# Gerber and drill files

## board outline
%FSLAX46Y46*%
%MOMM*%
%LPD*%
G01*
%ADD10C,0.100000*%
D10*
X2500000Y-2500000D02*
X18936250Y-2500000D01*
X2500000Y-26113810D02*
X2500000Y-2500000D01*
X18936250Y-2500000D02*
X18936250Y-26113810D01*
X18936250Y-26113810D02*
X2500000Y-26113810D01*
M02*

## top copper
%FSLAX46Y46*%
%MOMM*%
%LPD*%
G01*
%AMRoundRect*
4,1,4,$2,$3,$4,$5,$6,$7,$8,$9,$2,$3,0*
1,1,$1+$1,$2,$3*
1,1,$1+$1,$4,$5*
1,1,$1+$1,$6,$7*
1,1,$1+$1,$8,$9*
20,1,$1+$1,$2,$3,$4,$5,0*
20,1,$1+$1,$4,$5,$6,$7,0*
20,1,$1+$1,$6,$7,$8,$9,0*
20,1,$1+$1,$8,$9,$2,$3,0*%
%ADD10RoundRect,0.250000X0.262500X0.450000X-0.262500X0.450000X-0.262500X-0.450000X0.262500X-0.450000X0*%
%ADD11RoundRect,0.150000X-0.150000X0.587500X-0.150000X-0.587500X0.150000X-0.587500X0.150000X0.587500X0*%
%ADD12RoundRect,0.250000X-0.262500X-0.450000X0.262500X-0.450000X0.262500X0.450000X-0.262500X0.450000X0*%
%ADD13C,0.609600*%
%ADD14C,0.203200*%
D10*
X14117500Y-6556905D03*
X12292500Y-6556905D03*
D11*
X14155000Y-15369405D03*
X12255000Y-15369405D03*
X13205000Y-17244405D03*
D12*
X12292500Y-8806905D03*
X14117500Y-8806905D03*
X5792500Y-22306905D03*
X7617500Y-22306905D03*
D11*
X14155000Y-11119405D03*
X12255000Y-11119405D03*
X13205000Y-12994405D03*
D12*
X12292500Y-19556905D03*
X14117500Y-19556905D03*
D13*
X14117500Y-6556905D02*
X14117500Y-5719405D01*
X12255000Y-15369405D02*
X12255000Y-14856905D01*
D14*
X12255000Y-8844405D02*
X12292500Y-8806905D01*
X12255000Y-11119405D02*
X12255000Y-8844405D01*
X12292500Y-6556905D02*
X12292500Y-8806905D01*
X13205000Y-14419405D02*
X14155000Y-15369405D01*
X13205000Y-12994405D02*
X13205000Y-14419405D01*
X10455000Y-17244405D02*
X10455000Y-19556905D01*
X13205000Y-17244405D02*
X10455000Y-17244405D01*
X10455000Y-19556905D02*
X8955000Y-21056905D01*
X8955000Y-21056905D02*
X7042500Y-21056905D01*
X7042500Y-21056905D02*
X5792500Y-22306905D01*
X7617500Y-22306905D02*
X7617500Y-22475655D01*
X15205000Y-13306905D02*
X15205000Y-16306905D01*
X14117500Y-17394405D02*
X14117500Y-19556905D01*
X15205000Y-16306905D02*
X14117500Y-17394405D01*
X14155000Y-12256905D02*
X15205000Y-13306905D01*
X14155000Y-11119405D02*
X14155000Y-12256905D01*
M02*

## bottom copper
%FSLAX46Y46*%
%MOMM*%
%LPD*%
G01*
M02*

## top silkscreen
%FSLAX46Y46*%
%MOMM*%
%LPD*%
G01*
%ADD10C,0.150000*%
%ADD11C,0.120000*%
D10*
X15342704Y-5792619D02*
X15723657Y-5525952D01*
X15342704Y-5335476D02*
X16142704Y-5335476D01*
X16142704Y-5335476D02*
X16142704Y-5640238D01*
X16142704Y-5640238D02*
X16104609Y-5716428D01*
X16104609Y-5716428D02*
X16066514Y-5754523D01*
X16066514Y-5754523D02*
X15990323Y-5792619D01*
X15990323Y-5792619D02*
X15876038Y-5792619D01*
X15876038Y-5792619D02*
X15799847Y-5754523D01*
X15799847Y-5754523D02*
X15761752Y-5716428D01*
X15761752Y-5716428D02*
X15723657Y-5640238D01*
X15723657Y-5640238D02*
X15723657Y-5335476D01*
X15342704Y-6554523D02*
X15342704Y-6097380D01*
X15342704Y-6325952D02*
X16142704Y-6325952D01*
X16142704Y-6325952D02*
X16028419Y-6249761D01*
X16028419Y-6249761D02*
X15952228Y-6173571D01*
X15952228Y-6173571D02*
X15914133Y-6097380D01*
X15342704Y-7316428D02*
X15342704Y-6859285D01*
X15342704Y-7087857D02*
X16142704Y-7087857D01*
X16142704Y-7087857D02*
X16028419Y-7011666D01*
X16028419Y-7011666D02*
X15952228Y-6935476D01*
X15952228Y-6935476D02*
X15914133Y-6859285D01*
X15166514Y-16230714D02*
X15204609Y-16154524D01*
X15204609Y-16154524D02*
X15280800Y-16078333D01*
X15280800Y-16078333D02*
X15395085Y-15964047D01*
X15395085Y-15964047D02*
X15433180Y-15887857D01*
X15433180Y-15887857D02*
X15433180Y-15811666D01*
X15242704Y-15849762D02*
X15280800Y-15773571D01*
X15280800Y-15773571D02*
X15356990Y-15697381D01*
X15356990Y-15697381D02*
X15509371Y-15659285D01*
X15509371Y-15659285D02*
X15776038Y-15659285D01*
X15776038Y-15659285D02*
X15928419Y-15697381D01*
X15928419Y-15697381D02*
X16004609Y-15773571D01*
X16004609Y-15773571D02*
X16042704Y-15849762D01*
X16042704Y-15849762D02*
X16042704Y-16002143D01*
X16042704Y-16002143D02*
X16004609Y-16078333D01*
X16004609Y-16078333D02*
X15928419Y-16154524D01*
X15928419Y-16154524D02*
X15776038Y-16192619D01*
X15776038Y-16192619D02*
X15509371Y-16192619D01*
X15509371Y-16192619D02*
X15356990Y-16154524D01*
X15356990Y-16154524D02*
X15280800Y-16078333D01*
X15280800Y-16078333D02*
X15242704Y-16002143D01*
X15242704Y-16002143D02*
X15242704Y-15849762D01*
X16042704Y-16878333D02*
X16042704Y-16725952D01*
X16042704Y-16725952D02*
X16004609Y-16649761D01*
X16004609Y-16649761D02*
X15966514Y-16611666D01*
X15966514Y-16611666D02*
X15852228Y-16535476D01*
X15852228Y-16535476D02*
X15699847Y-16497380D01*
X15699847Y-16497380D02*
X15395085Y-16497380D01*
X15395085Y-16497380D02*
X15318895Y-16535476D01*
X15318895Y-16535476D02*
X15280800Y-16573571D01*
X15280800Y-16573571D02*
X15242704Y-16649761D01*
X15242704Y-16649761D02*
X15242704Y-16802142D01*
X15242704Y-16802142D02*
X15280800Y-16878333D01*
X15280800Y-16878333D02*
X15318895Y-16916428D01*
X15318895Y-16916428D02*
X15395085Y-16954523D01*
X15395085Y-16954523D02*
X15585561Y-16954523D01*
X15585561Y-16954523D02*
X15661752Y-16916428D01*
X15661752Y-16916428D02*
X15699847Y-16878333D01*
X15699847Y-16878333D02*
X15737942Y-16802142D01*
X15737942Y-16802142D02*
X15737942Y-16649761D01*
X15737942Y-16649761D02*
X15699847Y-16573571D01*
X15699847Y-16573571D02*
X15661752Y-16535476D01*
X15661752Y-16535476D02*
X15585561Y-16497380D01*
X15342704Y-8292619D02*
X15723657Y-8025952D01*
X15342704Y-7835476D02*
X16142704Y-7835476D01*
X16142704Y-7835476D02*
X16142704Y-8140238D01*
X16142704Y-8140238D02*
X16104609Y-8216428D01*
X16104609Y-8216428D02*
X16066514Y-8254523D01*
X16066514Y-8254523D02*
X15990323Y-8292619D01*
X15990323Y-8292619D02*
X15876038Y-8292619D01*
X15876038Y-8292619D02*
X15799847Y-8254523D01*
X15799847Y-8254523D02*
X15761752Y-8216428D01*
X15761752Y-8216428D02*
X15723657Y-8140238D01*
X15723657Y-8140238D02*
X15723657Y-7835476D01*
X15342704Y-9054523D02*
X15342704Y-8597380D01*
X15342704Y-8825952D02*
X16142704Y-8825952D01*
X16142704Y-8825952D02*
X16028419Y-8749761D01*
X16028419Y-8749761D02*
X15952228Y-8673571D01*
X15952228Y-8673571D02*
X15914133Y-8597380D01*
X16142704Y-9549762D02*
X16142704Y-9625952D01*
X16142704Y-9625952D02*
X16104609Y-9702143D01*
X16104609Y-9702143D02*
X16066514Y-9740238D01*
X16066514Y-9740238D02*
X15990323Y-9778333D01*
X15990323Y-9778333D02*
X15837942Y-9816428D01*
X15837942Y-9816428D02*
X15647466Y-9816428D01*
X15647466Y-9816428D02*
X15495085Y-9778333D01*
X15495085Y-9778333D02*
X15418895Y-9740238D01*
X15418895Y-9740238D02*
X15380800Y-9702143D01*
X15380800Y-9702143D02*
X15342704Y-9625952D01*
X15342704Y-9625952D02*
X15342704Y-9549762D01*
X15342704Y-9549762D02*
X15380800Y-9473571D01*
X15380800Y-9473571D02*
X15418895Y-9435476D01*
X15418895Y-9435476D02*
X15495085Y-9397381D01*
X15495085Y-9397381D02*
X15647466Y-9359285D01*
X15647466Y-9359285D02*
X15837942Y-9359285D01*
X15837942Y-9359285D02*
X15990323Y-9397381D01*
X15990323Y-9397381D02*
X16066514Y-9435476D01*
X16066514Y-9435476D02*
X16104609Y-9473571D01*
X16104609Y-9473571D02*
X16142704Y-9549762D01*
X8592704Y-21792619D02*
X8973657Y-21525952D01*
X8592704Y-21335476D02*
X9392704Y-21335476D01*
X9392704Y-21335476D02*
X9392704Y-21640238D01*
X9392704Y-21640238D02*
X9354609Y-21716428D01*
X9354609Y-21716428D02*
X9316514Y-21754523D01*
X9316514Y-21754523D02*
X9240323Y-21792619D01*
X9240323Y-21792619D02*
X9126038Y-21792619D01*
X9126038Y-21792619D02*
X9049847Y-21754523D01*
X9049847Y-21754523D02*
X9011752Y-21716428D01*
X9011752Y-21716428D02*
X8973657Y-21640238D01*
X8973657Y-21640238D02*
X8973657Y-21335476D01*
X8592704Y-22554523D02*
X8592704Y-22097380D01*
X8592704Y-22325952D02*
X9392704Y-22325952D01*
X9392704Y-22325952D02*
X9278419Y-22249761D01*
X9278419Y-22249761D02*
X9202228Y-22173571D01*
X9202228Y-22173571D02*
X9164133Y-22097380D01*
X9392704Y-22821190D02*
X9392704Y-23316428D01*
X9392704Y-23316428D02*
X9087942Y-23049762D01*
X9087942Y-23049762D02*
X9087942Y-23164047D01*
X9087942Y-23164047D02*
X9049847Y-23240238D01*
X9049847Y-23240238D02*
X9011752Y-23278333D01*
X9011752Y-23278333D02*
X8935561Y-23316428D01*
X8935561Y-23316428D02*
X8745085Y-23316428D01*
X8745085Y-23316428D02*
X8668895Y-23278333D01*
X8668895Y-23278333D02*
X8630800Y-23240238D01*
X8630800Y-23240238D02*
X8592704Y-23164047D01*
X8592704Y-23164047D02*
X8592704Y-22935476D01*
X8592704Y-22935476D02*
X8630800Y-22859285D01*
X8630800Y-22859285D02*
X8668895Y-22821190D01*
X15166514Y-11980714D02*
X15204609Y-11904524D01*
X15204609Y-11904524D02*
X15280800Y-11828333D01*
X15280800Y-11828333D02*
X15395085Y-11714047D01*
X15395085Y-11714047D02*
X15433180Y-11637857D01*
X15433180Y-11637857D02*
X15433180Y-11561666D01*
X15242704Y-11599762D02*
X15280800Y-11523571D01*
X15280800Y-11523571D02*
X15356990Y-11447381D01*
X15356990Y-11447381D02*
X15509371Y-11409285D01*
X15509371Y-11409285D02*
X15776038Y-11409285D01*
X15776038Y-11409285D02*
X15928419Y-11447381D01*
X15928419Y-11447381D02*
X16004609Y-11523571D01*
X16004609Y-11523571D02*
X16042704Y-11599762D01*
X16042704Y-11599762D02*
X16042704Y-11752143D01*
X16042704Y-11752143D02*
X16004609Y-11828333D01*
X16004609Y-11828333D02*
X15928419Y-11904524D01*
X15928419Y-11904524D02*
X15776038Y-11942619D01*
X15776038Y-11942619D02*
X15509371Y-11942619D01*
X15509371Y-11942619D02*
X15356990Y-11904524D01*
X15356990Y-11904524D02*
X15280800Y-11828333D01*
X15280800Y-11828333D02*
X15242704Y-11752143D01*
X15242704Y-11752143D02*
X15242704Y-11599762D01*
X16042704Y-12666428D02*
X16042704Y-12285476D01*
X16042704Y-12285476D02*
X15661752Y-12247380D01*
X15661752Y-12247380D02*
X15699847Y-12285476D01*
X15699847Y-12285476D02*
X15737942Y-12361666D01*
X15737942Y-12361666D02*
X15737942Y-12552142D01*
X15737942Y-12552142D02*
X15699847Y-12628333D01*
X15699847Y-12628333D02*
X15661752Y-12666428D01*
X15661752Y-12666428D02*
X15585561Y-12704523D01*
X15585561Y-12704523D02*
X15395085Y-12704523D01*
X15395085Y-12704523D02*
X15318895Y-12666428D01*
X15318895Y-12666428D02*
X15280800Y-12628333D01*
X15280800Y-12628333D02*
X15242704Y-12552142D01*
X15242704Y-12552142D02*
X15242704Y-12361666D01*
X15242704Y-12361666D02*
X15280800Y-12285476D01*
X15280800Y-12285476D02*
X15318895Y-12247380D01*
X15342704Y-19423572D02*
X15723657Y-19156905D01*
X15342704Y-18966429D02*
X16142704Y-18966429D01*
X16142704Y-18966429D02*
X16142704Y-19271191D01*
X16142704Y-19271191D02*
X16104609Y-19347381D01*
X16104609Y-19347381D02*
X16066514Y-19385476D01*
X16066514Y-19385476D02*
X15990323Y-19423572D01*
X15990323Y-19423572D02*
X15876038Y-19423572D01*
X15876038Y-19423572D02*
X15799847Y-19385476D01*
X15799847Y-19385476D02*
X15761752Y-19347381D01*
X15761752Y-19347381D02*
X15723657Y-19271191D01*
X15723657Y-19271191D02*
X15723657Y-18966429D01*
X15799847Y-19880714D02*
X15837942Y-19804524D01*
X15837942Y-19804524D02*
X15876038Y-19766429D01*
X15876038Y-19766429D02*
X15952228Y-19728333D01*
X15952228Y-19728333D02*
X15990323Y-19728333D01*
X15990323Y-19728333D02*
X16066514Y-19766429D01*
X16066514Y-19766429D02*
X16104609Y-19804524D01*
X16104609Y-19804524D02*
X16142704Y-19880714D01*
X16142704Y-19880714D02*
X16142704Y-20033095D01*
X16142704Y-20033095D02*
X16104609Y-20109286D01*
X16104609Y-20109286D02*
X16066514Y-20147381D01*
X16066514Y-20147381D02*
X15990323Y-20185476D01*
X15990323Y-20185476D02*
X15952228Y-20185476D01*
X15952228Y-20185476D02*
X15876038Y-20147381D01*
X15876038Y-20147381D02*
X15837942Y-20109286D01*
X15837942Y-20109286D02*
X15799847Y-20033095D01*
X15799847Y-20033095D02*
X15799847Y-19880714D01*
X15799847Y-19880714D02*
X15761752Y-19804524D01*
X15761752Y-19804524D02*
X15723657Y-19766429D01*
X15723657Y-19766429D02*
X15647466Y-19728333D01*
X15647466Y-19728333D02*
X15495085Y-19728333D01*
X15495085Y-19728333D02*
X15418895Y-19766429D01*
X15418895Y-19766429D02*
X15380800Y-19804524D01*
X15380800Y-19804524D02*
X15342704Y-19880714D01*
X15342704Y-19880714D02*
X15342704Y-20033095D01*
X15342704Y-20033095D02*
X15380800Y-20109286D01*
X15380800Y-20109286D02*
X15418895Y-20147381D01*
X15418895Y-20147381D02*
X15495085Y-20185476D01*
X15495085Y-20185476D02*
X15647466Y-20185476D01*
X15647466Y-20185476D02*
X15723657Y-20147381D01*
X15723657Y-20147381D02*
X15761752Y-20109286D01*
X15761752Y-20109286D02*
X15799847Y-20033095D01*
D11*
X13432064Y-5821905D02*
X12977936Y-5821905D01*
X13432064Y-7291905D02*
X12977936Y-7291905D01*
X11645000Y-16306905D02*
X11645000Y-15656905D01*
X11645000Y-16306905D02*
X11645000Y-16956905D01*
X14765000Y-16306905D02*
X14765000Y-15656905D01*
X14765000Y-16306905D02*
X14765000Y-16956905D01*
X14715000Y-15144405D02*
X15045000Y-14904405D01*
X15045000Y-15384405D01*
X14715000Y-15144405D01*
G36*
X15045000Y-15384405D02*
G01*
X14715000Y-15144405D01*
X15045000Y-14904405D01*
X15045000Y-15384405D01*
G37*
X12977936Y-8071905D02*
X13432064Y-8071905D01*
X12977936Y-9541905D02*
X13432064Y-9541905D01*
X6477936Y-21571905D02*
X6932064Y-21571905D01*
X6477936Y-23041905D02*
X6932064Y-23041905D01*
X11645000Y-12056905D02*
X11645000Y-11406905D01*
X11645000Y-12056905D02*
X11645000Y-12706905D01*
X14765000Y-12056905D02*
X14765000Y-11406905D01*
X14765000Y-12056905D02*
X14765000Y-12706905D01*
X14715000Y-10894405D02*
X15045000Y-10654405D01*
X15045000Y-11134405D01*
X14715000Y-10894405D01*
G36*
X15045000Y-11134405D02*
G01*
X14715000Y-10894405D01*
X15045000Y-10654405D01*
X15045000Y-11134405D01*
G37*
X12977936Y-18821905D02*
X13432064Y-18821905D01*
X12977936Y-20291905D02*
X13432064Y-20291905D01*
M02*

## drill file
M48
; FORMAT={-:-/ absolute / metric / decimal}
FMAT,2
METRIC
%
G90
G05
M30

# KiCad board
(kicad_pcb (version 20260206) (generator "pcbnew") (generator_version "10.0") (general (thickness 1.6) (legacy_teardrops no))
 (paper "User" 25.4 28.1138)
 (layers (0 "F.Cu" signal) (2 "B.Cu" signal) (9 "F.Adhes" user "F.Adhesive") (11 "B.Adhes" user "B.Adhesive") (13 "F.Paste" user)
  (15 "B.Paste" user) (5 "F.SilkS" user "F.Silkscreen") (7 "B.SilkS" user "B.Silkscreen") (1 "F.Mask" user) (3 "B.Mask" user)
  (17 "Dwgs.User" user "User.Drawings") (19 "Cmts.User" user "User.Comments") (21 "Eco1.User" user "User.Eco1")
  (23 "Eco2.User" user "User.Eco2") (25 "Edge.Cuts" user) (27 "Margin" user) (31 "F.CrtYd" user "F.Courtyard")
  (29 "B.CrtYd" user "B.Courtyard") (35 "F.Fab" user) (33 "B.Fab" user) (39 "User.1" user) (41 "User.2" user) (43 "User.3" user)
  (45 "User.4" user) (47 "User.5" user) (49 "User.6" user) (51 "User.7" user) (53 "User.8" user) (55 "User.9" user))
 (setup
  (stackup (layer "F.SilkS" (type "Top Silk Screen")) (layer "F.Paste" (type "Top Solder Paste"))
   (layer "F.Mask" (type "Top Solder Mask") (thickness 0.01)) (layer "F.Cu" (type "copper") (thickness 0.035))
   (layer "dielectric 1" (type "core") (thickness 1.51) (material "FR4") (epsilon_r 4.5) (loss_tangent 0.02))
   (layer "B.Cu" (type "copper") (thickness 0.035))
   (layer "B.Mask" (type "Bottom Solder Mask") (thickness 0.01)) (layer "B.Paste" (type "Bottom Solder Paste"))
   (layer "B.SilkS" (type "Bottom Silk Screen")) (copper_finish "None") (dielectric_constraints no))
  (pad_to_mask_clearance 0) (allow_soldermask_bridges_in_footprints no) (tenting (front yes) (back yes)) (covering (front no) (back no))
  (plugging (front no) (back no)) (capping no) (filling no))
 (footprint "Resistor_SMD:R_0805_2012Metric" (layer "F.Cu") (at 13.205 6.556905 180)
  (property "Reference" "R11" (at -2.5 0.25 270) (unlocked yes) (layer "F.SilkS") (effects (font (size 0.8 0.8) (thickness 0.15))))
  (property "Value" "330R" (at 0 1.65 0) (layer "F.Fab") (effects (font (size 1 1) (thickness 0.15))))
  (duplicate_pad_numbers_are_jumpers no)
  (fp_line (start -0.227064 0.735) (end 0.227064 0.735) (stroke (width 0.12) (type solid)) (layer "F.SilkS"))
  (fp_line (start -0.227064 -0.735) (end 0.227064 -0.735) (stroke (width 0.12) (type solid)) (layer "F.SilkS"))
  (pad "1" smd roundrect (at -0.9125 0 180) (size 1.025 1.4) (layers "F.Cu" "F.Mask" "F.Paste") (roundrect_rratio 0.243902) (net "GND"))
  (pad "2" smd roundrect (at 0.9125 0 180) (size 1.025 1.4) (layers "F.Cu" "F.Mask" "F.Paste") (roundrect_rratio 0.243902)
   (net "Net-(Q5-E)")))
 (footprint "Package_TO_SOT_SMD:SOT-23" (layer "F.Cu") (at 13.205 16.306905 -90)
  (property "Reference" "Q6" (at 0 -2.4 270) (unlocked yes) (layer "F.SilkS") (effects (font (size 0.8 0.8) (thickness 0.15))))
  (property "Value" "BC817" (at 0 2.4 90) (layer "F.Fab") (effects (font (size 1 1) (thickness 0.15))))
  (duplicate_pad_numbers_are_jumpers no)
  (fp_line (start 0 1.56) (end -0.65 1.56) (stroke (width 0.12) (type solid)) (layer "F.SilkS"))
  (fp_line (start 0 1.56) (end 0.65 1.56) (stroke (width 0.12) (type solid)) (layer "F.SilkS"))
  (fp_line (start 0 -1.56) (end -0.65 -1.56) (stroke (width 0.12) (type solid)) (layer "F.SilkS"))
  (fp_line (start 0 -1.56) (end 0.65 -1.56) (stroke (width 0.12) (type solid)) (layer "F.SilkS"))
  (fp_poly
   (pts (xy -1.1625 -1.51) (xy -1.4025 -1.84) (xy -0.9225 -1.84) (xy -1.1625 -1.51)) (stroke (width 0.12) (type solid)) (fill yes)
   (layer "F.SilkS"))
  (pad "1" smd roundrect (at -0.9375 -0.95 270) (size 1.475 0.6) (layers "F.Cu" "F.Mask" "F.Paste") (roundrect_rratio 0.25)
   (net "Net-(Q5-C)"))
  (pad "2" smd roundrect (at -0.9375 0.95 270) (size 1.475 0.6) (layers "F.Cu" "F.Mask" "F.Paste") (roundrect_rratio 0.25) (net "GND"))
  (pad "3" smd roundrect (at 0.9375 0 270) (size 1.475 0.6) (layers "F.Cu" "F.Mask" "F.Paste") (roundrect_rratio 0.25) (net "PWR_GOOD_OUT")))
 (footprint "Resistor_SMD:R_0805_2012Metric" (layer "F.Cu") (at 13.205 8.806905)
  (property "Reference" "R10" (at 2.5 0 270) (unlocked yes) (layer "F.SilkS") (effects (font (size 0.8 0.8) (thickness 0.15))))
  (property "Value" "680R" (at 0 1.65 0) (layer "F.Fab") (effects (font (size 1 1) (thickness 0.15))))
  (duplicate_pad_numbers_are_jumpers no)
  (fp_line (start -0.227064 -0.735) (end 0.227064 -0.735) (stroke (width 0.12) (type solid)) (layer "F.SilkS"))
  (fp_line (start -0.227064 0.735) (end 0.227064 0.735) (stroke (width 0.12) (type solid)) (layer "F.SilkS"))
  (pad "1" smd roundrect (at -0.9125 0) (size 1.025 1.4) (layers "F.Cu" "F.Mask" "F.Paste") (roundrect_rratio 0.243902) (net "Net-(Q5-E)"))
  (pad "2" smd roundrect (at 0.9125 0) (size 1.025 1.4) (layers "F.Cu" "F.Mask" "F.Paste") (roundrect_rratio 0.243902) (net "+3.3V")))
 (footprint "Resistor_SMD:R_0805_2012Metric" (layer "F.Cu") (at 6.705 22.306905)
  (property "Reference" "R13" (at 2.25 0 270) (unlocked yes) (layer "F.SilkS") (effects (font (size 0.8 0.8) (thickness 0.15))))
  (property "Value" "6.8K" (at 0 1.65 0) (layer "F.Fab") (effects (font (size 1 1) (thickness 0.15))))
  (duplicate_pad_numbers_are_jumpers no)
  (fp_line (start -0.227064 -0.735) (end 0.227064 -0.735) (stroke (width 0.12) (type solid)) (layer "F.SilkS"))
  (fp_line (start -0.227064 0.735) (end 0.227064 0.735) (stroke (width 0.12) (type solid)) (layer "F.SilkS"))
  (pad "1" smd roundrect (at -0.9125 0) (size 1.025 1.4) (layers "F.Cu" "F.Mask" "F.Paste") (roundrect_rratio 0.243902) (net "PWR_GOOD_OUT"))
  (pad "2" smd roundrect (at 0.9125 0) (size 1.025 1.4) (layers "F.Cu" "F.Mask" "F.Paste") (roundrect_rratio 0.243902) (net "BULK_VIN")))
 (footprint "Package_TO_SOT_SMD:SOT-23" (layer "F.Cu") (at 13.205 12.056905 -90)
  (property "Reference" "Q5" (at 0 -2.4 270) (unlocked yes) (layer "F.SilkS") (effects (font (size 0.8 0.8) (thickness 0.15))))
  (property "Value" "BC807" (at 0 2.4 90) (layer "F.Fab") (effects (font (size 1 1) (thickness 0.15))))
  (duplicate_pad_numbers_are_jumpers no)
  (fp_line (start 0 1.56) (end -0.65 1.56) (stroke (width 0.12) (type solid)) (layer "F.SilkS"))
  (fp_line (start 0 1.56) (end 0.65 1.56) (stroke (width 0.12) (type solid)) (layer "F.SilkS"))
  (fp_line (start 0 -1.56) (end -0.65 -1.56) (stroke (width 0.12) (type solid)) (layer "F.SilkS"))
  (fp_line (start 0 -1.56) (end 0.65 -1.56) (stroke (width 0.12) (type solid)) (layer "F.SilkS"))
  (fp_poly
   (pts (xy -1.1625 -1.51) (xy -1.4025 -1.84) (xy -0.9225 -1.84) (xy -1.1625 -1.51)) (stroke (width 0.12) (type solid)) (fill yes)
   (layer "F.SilkS"))
  (pad "1" smd roundrect (at -0.9375 -0.95 270) (size 1.475 0.6) (layers "F.Cu" "F.Mask" "F.Paste") (roundrect_rratio 0.25)
   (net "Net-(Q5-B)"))
  (pad "2" smd roundrect (at -0.9375 0.95 270) (size 1.475 0.6) (layers "F.Cu" "F.Mask" "F.Paste") (roundrect_rratio 0.25)
   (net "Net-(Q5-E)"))
  (pad "3" smd roundrect (at 0.9375 0 270) (size 1.475 0.6) (layers "F.Cu" "F.Mask" "F.Paste") (roundrect_rratio 0.25) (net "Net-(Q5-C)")))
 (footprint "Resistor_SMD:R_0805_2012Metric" (layer "F.Cu") (at 13.205 19.556905)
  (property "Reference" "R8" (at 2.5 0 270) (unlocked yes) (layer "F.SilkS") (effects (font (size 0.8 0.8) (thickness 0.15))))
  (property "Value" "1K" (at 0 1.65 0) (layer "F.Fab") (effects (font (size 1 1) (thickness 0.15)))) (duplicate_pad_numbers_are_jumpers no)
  (fp_line (start -0.227064 -0.735) (end 0.227064 -0.735) (stroke (width 0.12) (type solid)) (layer "F.SilkS"))
  (fp_line (start -0.227064 0.735) (end 0.227064 0.735) (stroke (width 0.12) (type solid)) (layer "F.SilkS"))
  (pad "1" smd roundrect (at -0.9125 0) (size 1.025 1.4) (layers "F.Cu" "F.Mask" "F.Paste") (roundrect_rratio 0.243902) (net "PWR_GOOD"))
  (pad "2" smd roundrect (at 0.9125 0) (size 1.025 1.4) (layers "F.Cu" "F.Mask" "F.Paste") (roundrect_rratio 0.243902) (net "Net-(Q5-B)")))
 (gr_line (start 2.5 2.5) (end 18.93625 2.5) (stroke (width 0.1) (type default)) (layer "Edge.Cuts"))
 (gr_line (start 2.5 26.11381) (end 2.5 2.5) (stroke (width 0.1) (type default)) (layer "Edge.Cuts"))
 (gr_line (start 18.93625 2.5) (end 18.93625 26.11381) (stroke (width 0.1) (type default)) (layer "Edge.Cuts"))
 (gr_line (start 18.93625 26.11381) (end 2.5 26.11381) (stroke (width 0.1) (type default)) (layer "Edge.Cuts"))
 (segment (start 14.1175 6.556905) (end 14.1175 5.719405) (width 0.6096) (layer "F.Cu") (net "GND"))
 (segment (start 12.255 15.369405) (end 12.255 14.856905) (width 0.6096) (layer "F.Cu") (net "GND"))
 (segment (start 12.255 8.844405) (end 12.2925 8.806905) (width 0.2032) (layer "F.Cu") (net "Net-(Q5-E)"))
 (segment (start 12.255 11.119405) (end 12.255 8.844405) (width 0.2032) (layer "F.Cu") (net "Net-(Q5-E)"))
 (segment (start 12.2925 6.556905) (end 12.2925 8.806905) (width 0.2032) (layer "F.Cu") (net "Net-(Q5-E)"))
 (segment (start 13.205 14.419405) (end 14.155 15.369405) (width 0.2032) (layer "F.Cu") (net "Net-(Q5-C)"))
 (segment (start 13.205 12.994405) (end 13.205 14.419405) (width 0.2032) (layer "F.Cu") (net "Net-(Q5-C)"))
 (segment (start 10.455 17.244405) (end 10.455 19.556905) (width 0.2032) (layer "F.Cu") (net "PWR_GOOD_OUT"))
 (segment (start 13.205 17.244405) (end 10.455 17.244405) (width 0.2032) (layer "F.Cu") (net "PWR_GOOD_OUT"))
 (segment (start 10.455 19.556905) (end 8.955 21.056905) (width 0.2032) (layer "F.Cu") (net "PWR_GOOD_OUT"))
 (segment (start 8.955 21.056905) (end 7.0425 21.056905) (width 0.2032) (layer "F.Cu") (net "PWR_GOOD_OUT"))
 (segment (start 7.0425 21.056905) (end 5.7925 22.306905) (width 0.2032) (layer "F.Cu") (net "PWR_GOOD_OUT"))
 (segment (start 7.6175 22.306905) (end 7.6175 22.475655) (width 0.2032) (layer "F.Cu") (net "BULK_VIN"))
 (segment (start 15.205 13.306905) (end 15.205 16.306905) (width 0.2032) (layer "F.Cu") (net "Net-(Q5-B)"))
 (segment (start 14.1175 17.394405) (end 14.1175 19.556905) (width 0.2032) (layer "F.Cu") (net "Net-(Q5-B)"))
 (segment (start 15.205 16.306905) (end 14.1175 17.394405) (width 0.2032) (layer "F.Cu") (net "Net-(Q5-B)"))
 (segment (start 14.155 12.256905) (end 15.205 13.306905) (width 0.2032) (layer "F.Cu") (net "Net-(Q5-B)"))
 (segment (start 14.155 11.119405) (end 14.155 12.256905) (width 0.2032) (layer "F.Cu") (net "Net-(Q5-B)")))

